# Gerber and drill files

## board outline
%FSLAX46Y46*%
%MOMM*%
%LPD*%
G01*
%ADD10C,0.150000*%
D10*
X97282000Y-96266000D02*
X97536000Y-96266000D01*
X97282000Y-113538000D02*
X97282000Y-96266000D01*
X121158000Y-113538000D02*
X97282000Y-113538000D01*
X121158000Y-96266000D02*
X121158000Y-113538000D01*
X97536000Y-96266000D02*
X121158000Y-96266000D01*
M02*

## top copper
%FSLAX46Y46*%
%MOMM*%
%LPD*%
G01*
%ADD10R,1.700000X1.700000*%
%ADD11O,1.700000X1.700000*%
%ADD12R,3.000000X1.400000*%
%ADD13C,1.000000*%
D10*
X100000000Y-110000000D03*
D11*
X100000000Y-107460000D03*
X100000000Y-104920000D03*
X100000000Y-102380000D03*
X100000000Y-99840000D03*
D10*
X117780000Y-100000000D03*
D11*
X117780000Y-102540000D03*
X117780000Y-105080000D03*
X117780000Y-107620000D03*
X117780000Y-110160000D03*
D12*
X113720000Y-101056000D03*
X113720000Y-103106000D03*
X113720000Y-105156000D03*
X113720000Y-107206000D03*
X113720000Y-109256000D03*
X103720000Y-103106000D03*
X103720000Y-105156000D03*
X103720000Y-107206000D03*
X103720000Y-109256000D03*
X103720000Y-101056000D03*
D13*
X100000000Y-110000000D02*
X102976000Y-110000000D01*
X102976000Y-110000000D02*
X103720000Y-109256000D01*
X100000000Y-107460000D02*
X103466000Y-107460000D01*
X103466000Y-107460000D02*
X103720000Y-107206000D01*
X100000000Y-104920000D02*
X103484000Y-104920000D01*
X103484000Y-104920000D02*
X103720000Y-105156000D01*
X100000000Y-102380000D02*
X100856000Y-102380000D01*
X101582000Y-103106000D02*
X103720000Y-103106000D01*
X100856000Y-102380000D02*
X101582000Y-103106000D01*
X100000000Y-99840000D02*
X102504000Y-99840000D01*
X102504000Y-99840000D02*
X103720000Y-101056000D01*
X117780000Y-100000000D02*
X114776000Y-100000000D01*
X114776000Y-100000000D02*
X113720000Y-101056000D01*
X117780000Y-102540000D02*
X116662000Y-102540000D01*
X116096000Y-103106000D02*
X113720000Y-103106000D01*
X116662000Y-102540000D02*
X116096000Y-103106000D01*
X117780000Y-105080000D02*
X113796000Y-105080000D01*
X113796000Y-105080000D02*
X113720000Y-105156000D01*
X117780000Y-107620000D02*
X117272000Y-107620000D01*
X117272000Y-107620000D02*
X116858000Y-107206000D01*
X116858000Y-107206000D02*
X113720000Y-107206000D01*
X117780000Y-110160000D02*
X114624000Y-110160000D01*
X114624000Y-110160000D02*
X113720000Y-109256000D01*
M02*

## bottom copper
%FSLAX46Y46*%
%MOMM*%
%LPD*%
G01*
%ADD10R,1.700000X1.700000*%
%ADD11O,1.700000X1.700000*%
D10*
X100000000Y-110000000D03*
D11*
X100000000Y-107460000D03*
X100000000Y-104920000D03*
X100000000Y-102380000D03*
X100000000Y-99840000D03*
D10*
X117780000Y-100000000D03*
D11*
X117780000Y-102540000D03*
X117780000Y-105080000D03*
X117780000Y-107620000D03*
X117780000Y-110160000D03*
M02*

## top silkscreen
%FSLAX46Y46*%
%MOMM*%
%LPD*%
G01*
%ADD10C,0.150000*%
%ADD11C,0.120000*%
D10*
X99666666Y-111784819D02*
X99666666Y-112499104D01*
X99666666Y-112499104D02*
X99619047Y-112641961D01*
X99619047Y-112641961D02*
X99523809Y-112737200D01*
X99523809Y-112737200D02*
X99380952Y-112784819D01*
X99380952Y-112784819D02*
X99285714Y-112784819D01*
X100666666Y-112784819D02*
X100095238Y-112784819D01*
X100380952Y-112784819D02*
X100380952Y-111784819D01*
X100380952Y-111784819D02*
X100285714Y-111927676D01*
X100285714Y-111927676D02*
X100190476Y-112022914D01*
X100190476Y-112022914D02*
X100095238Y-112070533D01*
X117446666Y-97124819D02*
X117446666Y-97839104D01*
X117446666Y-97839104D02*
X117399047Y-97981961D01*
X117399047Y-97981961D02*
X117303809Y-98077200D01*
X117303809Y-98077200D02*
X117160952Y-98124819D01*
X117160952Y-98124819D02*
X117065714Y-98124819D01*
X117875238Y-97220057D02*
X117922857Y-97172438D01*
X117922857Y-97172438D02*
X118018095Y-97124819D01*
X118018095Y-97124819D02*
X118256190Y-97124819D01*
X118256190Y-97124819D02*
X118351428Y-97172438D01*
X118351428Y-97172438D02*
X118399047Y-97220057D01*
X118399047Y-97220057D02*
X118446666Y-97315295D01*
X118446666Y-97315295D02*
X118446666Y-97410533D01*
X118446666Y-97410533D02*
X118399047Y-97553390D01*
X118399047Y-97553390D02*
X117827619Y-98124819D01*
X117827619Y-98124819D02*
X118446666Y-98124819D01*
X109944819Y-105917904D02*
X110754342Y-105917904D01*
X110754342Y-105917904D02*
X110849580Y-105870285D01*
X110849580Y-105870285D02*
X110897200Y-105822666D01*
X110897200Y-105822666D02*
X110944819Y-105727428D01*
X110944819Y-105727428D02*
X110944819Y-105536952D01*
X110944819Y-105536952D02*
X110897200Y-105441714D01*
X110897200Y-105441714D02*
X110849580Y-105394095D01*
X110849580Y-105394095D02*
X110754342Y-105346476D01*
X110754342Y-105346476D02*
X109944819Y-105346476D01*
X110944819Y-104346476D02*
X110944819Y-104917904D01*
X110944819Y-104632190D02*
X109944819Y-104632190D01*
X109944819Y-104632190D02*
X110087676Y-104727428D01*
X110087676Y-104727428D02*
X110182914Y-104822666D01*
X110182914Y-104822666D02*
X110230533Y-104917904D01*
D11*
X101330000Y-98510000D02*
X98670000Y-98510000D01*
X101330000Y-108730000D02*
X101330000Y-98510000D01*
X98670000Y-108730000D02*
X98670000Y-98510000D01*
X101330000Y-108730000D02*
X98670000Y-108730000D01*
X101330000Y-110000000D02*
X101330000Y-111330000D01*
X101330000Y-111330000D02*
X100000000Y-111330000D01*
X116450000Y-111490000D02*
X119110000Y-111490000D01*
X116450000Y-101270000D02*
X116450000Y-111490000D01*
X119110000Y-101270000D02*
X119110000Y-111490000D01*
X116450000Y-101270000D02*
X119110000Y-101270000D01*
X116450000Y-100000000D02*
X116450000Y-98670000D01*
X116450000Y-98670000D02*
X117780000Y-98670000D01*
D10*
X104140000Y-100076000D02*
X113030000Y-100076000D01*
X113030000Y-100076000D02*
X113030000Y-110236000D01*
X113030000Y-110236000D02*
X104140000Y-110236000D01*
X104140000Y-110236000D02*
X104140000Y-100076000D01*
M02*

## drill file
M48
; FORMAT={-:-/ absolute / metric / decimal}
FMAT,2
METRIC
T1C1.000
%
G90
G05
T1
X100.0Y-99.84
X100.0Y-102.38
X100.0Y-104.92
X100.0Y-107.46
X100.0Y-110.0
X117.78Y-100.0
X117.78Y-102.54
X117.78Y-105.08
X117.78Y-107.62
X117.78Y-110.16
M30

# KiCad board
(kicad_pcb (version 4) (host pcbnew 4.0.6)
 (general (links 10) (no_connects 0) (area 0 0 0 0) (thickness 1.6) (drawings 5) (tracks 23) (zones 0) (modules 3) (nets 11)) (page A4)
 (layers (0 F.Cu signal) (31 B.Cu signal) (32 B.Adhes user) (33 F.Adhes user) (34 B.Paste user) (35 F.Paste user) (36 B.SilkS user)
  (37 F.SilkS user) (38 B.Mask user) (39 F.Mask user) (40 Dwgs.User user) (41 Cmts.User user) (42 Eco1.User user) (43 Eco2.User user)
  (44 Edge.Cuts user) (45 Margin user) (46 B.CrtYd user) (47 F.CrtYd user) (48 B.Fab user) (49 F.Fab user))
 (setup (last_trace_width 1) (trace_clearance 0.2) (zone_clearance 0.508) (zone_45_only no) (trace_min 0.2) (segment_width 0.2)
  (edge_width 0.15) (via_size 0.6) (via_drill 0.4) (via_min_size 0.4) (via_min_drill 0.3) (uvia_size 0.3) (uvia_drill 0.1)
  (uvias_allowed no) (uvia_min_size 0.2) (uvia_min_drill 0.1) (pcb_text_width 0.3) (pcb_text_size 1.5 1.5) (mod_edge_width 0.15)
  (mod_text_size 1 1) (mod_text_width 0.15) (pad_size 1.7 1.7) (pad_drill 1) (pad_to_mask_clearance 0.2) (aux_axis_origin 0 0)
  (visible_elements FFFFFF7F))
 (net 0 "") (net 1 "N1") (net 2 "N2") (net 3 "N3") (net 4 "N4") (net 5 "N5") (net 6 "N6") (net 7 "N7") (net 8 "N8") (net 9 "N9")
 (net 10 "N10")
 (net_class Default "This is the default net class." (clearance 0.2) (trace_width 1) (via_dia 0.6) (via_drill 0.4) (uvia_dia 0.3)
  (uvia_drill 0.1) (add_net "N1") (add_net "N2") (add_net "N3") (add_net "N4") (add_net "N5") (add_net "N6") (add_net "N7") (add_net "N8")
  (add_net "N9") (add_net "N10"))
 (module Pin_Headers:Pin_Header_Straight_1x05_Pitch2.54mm (layer F.Cu) (at 100 110 180)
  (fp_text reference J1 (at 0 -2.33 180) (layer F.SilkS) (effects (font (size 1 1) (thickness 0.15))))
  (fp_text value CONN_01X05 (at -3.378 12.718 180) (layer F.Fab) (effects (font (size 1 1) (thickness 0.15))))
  (fp_line (start -1.33 11.49) (end 1.33 11.49) (layer F.SilkS) (width 0.12))
  (fp_line (start -1.33 1.27) (end -1.33 11.49) (layer F.SilkS) (width 0.12))
  (fp_line (start 1.33 1.27) (end 1.33 11.49) (layer F.SilkS) (width 0.12))
  (fp_line (start -1.33 1.27) (end 1.33 1.27) (layer F.SilkS) (width 0.12))
  (fp_line (start -1.33 0) (end -1.33 -1.33) (layer F.SilkS) (width 0.12))
  (fp_line (start -1.33 -1.33) (end 0 -1.33) (layer F.SilkS) (width 0.12))
  (pad 1 thru_hole rect (at 0 0 180) (size 1.7 1.7) (drill 1) (layers *.Cu *.Mask) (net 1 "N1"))
  (pad 2 thru_hole oval (at 0 2.54 180) (size 1.7 1.7) (drill 1) (layers *.Cu *.Mask) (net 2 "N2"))
  (pad 3 thru_hole oval (at 0 5.08 180) (size 1.7 1.7) (drill 1) (layers *.Cu *.Mask) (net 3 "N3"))
  (pad 4 thru_hole oval (at 0 7.62 180) (size 1.7 1.7) (drill 1) (layers *.Cu *.Mask) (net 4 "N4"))
  (pad 5 thru_hole oval (at 0 10.16 180) (size 1.7 1.7) (drill 1) (layers *.Cu *.Mask) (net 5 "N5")))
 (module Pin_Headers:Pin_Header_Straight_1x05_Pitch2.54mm (layer F.Cu) (at 117.78 100)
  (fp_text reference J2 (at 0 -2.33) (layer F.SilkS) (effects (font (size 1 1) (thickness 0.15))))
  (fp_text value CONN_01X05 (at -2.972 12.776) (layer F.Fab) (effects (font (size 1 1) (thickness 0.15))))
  (fp_line (start -1.33 11.49) (end 1.33 11.49) (layer F.SilkS) (width 0.12))
  (fp_line (start -1.33 1.27) (end -1.33 11.49) (layer F.SilkS) (width 0.12))
  (fp_line (start 1.33 1.27) (end 1.33 11.49) (layer F.SilkS) (width 0.12))
  (fp_line (start -1.33 1.27) (end 1.33 1.27) (layer F.SilkS) (width 0.12))
  (fp_line (start -1.33 0) (end -1.33 -1.33) (layer F.SilkS) (width 0.12))
  (fp_line (start -1.33 -1.33) (end 0 -1.33) (layer F.SilkS) (width 0.12))
  (pad 1 thru_hole rect (at 0 0) (size 1.7 1.7) (drill 1) (layers *.Cu *.Mask) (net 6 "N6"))
  (pad 2 thru_hole oval (at 0 2.54) (size 1.7 1.7) (drill 1) (layers *.Cu *.Mask) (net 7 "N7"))
  (pad 3 thru_hole oval (at 0 5.08) (size 1.7 1.7) (drill 1) (layers *.Cu *.Mask) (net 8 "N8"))
  (pad 4 thru_hole oval (at 0 7.62) (size 1.7 1.7) (drill 1) (layers *.Cu *.Mask) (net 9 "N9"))
  (pad 5 thru_hole oval (at 0 10.16) (size 1.7 1.7) (drill 1) (layers *.Cu *.Mask) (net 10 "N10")))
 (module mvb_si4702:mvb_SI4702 (layer F.Cu) (at 109.22 105.156)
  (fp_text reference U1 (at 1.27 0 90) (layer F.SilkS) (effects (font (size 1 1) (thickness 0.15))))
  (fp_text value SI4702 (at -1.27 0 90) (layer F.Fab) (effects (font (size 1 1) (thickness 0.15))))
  (fp_line (start -5.08 -5.08) (end 3.81 -5.08) (layer F.SilkS) (width 0.15))
  (fp_line (start 3.81 -5.08) (end 3.81 5.08) (layer F.SilkS) (width 0.15))
  (fp_line (start 3.81 5.08) (end -5.08 5.08) (layer F.SilkS) (width 0.15))
  (fp_line (start -5.08 5.08) (end -5.08 -5.08) (layer F.SilkS) (width 0.15))
  (pad 10 smd rect (at 4.5 -4.1) (size 3 1.4) (layers F.Cu F.Paste F.Mask) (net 6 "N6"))
  (pad 9 smd rect (at 4.5 -2.05) (size 3 1.4) (layers F.Cu F.Paste F.Mask) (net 7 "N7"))
  (pad 8 smd rect (at 4.5 0) (size 3 1.4) (layers F.Cu F.Paste F.Mask) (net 8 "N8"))
  (pad 7 smd rect (at 4.5 2.05) (size 3 1.4) (layers F.Cu F.Paste F.Mask) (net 9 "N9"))
  (pad 6 smd rect (at 4.5 4.1) (size 3 1.4) (layers F.Cu F.Paste F.Mask) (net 10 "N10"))
  (pad 2 smd rect (at -5.5 -2.05) (size 3 1.4) (layers F.Cu F.Paste F.Mask) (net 4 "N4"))
  (pad 3 smd rect (at -5.5 0) (size 3 1.4) (layers F.Cu F.Paste F.Mask) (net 3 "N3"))
  (pad 4 smd rect (at -5.5 2.05) (size 3 1.4) (layers F.Cu F.Paste F.Mask) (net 2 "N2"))
  (pad 5 smd rect (at -5.5 4.1) (size 3 1.4) (layers F.Cu F.Paste F.Mask) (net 1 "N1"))
  (pad 1 smd rect (at -5.5 -4.1) (size 3 1.4) (layers F.Cu F.Paste F.Mask) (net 5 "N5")))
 (gr_line (start 97.282 96.266) (end 97.536 96.266) (angle 90) (layer Edge.Cuts) (width 0.15))
 (gr_line (start 97.282 113.538) (end 97.282 96.266) (angle 90) (layer Edge.Cuts) (width 0.15))
 (gr_line (start 121.158 113.538) (end 97.282 113.538) (angle 90) (layer Edge.Cuts) (width 0.15))
 (gr_line (start 121.158 96.266) (end 121.158 113.538) (angle 90) (layer Edge.Cuts) (width 0.15))
 (gr_line (start 97.536 96.266) (end 121.158 96.266) (angle 90) (layer Edge.Cuts) (width 0.15))
 (segment (start 100 110) (end 102.976 110) (width 1) (layer F.Cu) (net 1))
 (segment (start 102.976 110) (end 103.72 109.256) (width 1) (layer F.Cu) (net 1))
 (segment (start 100 107.46) (end 103.466 107.46) (width 1) (layer F.Cu) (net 2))
 (segment (start 103.466 107.46) (end 103.72 107.206) (width 1) (layer F.Cu) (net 2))
 (segment (start 100 104.92) (end 103.484 104.92) (width 1) (layer F.Cu) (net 3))
 (segment (start 103.484 104.92) (end 103.72 105.156) (width 1) (layer F.Cu) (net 3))
 (segment (start 100 102.38) (end 100.856 102.38) (width 1) (layer F.Cu) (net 4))
 (segment (start 101.582 103.106) (end 103.72 103.106) (width 1) (layer F.Cu) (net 4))
 (segment (start 100.856 102.38) (end 101.582 103.106) (width 1) (layer F.Cu) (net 4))
 (segment (start 100 99.84) (end 102.504 99.84) (width 1) (layer F.Cu) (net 5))
 (segment (start 102.504 99.84) (end 103.72 101.056) (width 1) (layer F.Cu) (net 5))
 (segment (start 117.78 100) (end 114.776 100) (width 1) (layer F.Cu) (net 6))
 (segment (start 114.776 100) (end 113.72 101.056) (width 1) (layer F.Cu) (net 6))
 (segment (start 117.78 102.54) (end 116.662 102.54) (width 1) (layer F.Cu) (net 7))
 (segment (start 116.096 103.106) (end 113.72 103.106) (width 1) (layer F.Cu) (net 7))
 (segment (start 116.662 102.54) (end 116.096 103.106) (width 1) (layer F.Cu) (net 7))
 (segment (start 117.78 105.08) (end 113.796 105.08) (width 1) (layer F.Cu) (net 8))
 (segment (start 113.796 105.08) (end 113.72 105.156) (width 1) (layer F.Cu) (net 8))
 (segment (start 117.78 107.62) (end 117.272 107.62) (width 1) (layer F.Cu) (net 9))
 (segment (start 117.272 107.62) (end 116.858 107.206) (width 1) (layer F.Cu) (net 9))
 (segment (start 116.858 107.206) (end 113.72 107.206) (width 1) (layer F.Cu) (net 9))
 (segment (start 117.78 110.16) (end 114.624 110.16) (width 1) (layer F.Cu) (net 10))
 (segment (start 114.624 110.16) (end 113.72 109.256) (width 1) (layer F.Cu) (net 10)))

